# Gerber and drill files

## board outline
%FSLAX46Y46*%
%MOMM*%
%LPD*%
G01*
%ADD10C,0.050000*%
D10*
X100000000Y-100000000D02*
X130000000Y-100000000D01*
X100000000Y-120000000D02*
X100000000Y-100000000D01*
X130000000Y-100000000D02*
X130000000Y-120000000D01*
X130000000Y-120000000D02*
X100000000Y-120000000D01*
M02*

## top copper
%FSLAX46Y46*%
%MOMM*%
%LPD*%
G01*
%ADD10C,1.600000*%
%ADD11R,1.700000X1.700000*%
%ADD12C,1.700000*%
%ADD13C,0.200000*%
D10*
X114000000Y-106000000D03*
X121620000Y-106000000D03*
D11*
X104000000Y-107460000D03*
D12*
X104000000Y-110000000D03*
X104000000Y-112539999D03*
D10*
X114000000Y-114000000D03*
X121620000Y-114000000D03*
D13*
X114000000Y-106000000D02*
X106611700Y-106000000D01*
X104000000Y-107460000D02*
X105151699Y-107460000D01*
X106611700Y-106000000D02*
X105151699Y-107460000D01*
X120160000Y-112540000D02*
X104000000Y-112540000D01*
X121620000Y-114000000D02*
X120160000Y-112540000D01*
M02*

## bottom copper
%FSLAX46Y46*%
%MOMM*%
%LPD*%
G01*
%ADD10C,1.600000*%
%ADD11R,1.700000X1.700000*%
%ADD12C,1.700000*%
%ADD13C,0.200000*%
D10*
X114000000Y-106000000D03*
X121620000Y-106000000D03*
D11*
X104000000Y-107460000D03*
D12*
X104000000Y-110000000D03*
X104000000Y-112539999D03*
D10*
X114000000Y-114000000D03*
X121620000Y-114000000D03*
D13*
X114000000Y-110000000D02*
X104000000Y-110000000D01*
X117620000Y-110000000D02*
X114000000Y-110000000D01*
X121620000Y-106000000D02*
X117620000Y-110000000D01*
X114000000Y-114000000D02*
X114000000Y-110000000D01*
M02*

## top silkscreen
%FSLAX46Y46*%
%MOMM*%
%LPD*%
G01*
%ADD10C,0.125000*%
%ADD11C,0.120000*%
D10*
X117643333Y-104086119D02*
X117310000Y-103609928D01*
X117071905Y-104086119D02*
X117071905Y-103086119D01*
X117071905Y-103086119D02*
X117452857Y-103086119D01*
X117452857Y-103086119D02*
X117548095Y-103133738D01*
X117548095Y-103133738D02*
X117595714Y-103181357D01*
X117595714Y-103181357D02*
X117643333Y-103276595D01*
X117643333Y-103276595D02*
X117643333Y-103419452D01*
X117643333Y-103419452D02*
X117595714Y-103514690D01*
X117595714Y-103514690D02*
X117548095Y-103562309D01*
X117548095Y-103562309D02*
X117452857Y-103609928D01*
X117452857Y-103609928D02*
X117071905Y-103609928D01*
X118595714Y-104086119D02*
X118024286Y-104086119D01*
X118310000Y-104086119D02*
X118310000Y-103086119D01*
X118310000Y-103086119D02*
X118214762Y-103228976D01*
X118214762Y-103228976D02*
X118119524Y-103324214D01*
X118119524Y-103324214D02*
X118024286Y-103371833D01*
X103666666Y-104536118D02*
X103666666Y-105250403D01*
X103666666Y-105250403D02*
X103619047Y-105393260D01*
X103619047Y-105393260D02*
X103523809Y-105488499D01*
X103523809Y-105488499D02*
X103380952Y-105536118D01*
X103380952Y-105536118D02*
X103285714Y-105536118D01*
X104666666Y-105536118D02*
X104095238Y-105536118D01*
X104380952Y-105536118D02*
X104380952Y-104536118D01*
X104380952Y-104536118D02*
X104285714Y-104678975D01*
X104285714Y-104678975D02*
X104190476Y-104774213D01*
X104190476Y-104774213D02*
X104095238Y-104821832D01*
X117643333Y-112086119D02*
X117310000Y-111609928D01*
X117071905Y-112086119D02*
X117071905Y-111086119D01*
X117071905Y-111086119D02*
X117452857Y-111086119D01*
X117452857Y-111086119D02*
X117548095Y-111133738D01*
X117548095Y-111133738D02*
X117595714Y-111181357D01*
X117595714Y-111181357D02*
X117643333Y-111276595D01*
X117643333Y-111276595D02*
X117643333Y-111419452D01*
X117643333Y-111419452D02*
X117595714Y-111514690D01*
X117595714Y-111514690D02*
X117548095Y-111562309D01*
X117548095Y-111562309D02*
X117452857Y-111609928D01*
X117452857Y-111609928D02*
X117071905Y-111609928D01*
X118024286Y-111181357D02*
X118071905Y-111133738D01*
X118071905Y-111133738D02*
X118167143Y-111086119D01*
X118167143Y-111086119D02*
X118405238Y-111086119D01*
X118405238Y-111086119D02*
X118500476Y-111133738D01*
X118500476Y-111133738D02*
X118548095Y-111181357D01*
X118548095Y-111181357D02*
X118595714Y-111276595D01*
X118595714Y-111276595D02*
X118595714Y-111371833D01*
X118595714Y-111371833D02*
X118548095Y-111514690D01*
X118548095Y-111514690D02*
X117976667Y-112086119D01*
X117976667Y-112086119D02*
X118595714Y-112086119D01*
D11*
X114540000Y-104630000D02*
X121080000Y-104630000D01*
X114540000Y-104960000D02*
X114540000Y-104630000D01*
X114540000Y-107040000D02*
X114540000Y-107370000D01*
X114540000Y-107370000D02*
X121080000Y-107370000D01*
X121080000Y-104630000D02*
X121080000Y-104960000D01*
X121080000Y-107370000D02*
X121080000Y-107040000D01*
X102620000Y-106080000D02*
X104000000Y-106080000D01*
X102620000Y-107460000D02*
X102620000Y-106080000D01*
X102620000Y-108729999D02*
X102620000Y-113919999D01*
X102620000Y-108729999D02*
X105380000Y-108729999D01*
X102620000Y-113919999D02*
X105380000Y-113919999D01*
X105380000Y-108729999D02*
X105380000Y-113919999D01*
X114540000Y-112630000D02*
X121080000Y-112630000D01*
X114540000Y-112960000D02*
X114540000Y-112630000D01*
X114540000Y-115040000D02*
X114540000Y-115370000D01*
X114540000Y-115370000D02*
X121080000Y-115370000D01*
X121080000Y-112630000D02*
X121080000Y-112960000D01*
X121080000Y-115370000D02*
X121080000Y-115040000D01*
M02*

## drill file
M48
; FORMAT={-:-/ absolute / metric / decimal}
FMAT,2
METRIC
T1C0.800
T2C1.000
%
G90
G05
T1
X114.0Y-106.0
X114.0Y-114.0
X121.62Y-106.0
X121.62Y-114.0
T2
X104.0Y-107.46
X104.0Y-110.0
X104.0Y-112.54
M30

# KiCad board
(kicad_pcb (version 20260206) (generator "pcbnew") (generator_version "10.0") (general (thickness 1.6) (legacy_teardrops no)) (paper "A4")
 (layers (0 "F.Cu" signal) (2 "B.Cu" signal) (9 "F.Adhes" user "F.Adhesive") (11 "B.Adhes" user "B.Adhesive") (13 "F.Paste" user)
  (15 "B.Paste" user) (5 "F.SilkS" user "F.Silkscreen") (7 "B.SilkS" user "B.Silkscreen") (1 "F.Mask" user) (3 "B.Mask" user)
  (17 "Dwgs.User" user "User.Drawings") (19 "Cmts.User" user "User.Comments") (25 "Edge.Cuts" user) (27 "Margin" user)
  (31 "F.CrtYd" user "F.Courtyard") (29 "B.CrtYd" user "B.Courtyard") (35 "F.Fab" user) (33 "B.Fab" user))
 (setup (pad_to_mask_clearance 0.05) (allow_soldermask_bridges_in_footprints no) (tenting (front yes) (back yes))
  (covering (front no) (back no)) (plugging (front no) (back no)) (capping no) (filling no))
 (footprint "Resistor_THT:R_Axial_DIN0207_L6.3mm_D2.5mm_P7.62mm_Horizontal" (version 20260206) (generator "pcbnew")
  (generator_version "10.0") (layer "F.Cu") (at 114 106)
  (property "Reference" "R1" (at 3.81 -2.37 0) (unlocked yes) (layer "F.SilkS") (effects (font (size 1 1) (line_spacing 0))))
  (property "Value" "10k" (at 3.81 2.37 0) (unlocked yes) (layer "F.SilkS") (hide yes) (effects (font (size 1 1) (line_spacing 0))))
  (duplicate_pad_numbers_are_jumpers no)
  (fp_line (start 0.54 -1.37) (end 7.08 -1.37) (stroke (width 0.12) (type default)) (layer "F.SilkS"))
  (fp_line (start 0.54 -1.04) (end 0.54 -1.37) (stroke (width 0.12) (type default)) (layer "F.SilkS"))
  (fp_line (start 0.54 1.04) (end 0.54 1.37) (stroke (width 0.12) (type default)) (layer "F.SilkS"))
  (fp_line (start 0.54 1.37) (end 7.08 1.37) (stroke (width 0.12) (type default)) (layer "F.SilkS"))
  (fp_line (start 7.08 -1.37) (end 7.08 -1.04) (stroke (width 0.12) (type default)) (layer "F.SilkS"))
  (fp_line (start 7.08 1.37) (end 7.08 1.04) (stroke (width 0.12) (type default)) (layer "F.SilkS"))
  (pad "1" thru_hole circle (at 0 0) (size 1.6 1.6) (drill 0.8) (layers "*.Cu" "*.Mask") (remove_unused_layers no) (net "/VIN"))
  (pad "2" thru_hole circle (at 7.62 0) (size 1.6 1.6) (drill 0.8) (layers "*.Cu" "*.Mask") (remove_unused_layers no) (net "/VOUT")))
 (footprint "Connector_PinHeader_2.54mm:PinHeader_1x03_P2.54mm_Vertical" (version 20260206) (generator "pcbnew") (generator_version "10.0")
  (layer "F.Cu") (at 104 107.46)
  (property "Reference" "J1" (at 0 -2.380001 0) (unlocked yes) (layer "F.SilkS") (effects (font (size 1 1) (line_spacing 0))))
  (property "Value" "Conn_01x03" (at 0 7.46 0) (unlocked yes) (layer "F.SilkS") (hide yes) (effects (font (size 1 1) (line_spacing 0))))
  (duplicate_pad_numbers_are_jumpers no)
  (fp_line (start -1.38 -1.38) (end 0 -1.38) (stroke (width 0.12) (type default)) (layer "F.SilkS"))
  (fp_line (start -1.38 0) (end -1.38 -1.38) (stroke (width 0.12) (type default)) (layer "F.SilkS"))
  (fp_line (start -1.38 1.269999) (end -1.38 6.459999) (stroke (width 0.12) (type default)) (layer "F.SilkS"))
  (fp_line (start -1.38 1.269999) (end 1.38 1.269999) (stroke (width 0.12) (type default)) (layer "F.SilkS"))
  (fp_line (start -1.38 6.459999) (end 1.38 6.459999) (stroke (width 0.12) (type default)) (layer "F.SilkS"))
  (fp_line (start 1.38 1.269999) (end 1.38 6.459999) (stroke (width 0.12) (type default)) (layer "F.SilkS"))
  (pad "1" thru_hole rect (at 0 0) (size 1.7 1.7) (drill 1) (layers "*.Cu" "*.Mask") (remove_unused_layers no) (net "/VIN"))
  (pad "2" thru_hole circle (at 0 2.54) (size 1.7 1.7) (drill 1) (layers "*.Cu" "*.Mask") (remove_unused_layers no) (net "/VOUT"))
  (pad "3" thru_hole circle (at 0 5.079999) (size 1.7 1.7) (drill 1) (layers "*.Cu" "*.Mask") (remove_unused_layers no) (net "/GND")))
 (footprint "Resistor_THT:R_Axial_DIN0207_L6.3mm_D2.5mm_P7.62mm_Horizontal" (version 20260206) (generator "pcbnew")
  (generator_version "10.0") (layer "F.Cu") (at 114 114)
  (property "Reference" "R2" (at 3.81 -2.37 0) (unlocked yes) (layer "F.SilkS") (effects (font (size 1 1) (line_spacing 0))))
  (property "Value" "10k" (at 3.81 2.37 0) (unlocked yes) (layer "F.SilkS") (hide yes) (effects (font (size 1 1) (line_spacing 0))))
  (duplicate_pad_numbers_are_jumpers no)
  (fp_line (start 0.54 -1.37) (end 7.08 -1.37) (stroke (width 0.12) (type default)) (layer "F.SilkS"))
  (fp_line (start 0.54 -1.04) (end 0.54 -1.37) (stroke (width 0.12) (type default)) (layer "F.SilkS"))
  (fp_line (start 0.54 1.04) (end 0.54 1.37) (stroke (width 0.12) (type default)) (layer "F.SilkS"))
  (fp_line (start 0.54 1.37) (end 7.08 1.37) (stroke (width 0.12) (type default)) (layer "F.SilkS"))
  (fp_line (start 7.08 -1.37) (end 7.08 -1.04) (stroke (width 0.12) (type default)) (layer "F.SilkS"))
  (fp_line (start 7.08 1.37) (end 7.08 1.04) (stroke (width 0.12) (type default)) (layer "F.SilkS"))
  (pad "1" thru_hole circle (at 0 0) (size 1.6 1.6) (drill 0.8) (layers "*.Cu" "*.Mask") (remove_unused_layers no) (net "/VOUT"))
  (pad "2" thru_hole circle (at 7.62 0) (size 1.6 1.6) (drill 0.8) (layers "*.Cu" "*.Mask") (remove_unused_layers no) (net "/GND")))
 (gr_line (start 100 100) (end 130 100) (stroke (width 0.05) (type default)) (layer "Edge.Cuts"))
 (gr_line (start 100 120) (end 100 100) (stroke (width 0.05) (type default)) (layer "Edge.Cuts"))
 (gr_line (start 130 100) (end 130 120) (stroke (width 0.05) (type default)) (layer "Edge.Cuts"))
 (gr_line (start 130 120) (end 100 120) (stroke (width 0.05) (type default)) (layer "Edge.Cuts"))
 (segment (start 114 106) (end 106.6117 106) (width 0.2) (layer "F.Cu") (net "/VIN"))
 (segment (start 104 107.46) (end 105.151699 107.46) (width 0.2) (layer "F.Cu") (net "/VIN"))
 (segment (start 106.6117 106) (end 105.151699 107.46) (width 0.2) (layer "F.Cu") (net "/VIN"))
 (segment (start 114 110) (end 104 110) (width 0.2) (layer "B.Cu") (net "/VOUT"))
 (segment (start 117.62 110) (end 114 110) (width 0.2) (layer "B.Cu") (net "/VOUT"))
 (segment (start 121.62 106) (end 117.62 110) (width 0.2) (layer "B.Cu") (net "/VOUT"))
 (segment (start 114 114) (end 114 110) (width 0.2) (layer "B.Cu") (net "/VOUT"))
 (segment (start 120.16 112.54) (end 104 112.54) (width 0.2) (layer "F.Cu") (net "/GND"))
 (segment (start 121.62 114) (end 120.16 112.54) (width 0.2) (layer "F.Cu") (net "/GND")))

